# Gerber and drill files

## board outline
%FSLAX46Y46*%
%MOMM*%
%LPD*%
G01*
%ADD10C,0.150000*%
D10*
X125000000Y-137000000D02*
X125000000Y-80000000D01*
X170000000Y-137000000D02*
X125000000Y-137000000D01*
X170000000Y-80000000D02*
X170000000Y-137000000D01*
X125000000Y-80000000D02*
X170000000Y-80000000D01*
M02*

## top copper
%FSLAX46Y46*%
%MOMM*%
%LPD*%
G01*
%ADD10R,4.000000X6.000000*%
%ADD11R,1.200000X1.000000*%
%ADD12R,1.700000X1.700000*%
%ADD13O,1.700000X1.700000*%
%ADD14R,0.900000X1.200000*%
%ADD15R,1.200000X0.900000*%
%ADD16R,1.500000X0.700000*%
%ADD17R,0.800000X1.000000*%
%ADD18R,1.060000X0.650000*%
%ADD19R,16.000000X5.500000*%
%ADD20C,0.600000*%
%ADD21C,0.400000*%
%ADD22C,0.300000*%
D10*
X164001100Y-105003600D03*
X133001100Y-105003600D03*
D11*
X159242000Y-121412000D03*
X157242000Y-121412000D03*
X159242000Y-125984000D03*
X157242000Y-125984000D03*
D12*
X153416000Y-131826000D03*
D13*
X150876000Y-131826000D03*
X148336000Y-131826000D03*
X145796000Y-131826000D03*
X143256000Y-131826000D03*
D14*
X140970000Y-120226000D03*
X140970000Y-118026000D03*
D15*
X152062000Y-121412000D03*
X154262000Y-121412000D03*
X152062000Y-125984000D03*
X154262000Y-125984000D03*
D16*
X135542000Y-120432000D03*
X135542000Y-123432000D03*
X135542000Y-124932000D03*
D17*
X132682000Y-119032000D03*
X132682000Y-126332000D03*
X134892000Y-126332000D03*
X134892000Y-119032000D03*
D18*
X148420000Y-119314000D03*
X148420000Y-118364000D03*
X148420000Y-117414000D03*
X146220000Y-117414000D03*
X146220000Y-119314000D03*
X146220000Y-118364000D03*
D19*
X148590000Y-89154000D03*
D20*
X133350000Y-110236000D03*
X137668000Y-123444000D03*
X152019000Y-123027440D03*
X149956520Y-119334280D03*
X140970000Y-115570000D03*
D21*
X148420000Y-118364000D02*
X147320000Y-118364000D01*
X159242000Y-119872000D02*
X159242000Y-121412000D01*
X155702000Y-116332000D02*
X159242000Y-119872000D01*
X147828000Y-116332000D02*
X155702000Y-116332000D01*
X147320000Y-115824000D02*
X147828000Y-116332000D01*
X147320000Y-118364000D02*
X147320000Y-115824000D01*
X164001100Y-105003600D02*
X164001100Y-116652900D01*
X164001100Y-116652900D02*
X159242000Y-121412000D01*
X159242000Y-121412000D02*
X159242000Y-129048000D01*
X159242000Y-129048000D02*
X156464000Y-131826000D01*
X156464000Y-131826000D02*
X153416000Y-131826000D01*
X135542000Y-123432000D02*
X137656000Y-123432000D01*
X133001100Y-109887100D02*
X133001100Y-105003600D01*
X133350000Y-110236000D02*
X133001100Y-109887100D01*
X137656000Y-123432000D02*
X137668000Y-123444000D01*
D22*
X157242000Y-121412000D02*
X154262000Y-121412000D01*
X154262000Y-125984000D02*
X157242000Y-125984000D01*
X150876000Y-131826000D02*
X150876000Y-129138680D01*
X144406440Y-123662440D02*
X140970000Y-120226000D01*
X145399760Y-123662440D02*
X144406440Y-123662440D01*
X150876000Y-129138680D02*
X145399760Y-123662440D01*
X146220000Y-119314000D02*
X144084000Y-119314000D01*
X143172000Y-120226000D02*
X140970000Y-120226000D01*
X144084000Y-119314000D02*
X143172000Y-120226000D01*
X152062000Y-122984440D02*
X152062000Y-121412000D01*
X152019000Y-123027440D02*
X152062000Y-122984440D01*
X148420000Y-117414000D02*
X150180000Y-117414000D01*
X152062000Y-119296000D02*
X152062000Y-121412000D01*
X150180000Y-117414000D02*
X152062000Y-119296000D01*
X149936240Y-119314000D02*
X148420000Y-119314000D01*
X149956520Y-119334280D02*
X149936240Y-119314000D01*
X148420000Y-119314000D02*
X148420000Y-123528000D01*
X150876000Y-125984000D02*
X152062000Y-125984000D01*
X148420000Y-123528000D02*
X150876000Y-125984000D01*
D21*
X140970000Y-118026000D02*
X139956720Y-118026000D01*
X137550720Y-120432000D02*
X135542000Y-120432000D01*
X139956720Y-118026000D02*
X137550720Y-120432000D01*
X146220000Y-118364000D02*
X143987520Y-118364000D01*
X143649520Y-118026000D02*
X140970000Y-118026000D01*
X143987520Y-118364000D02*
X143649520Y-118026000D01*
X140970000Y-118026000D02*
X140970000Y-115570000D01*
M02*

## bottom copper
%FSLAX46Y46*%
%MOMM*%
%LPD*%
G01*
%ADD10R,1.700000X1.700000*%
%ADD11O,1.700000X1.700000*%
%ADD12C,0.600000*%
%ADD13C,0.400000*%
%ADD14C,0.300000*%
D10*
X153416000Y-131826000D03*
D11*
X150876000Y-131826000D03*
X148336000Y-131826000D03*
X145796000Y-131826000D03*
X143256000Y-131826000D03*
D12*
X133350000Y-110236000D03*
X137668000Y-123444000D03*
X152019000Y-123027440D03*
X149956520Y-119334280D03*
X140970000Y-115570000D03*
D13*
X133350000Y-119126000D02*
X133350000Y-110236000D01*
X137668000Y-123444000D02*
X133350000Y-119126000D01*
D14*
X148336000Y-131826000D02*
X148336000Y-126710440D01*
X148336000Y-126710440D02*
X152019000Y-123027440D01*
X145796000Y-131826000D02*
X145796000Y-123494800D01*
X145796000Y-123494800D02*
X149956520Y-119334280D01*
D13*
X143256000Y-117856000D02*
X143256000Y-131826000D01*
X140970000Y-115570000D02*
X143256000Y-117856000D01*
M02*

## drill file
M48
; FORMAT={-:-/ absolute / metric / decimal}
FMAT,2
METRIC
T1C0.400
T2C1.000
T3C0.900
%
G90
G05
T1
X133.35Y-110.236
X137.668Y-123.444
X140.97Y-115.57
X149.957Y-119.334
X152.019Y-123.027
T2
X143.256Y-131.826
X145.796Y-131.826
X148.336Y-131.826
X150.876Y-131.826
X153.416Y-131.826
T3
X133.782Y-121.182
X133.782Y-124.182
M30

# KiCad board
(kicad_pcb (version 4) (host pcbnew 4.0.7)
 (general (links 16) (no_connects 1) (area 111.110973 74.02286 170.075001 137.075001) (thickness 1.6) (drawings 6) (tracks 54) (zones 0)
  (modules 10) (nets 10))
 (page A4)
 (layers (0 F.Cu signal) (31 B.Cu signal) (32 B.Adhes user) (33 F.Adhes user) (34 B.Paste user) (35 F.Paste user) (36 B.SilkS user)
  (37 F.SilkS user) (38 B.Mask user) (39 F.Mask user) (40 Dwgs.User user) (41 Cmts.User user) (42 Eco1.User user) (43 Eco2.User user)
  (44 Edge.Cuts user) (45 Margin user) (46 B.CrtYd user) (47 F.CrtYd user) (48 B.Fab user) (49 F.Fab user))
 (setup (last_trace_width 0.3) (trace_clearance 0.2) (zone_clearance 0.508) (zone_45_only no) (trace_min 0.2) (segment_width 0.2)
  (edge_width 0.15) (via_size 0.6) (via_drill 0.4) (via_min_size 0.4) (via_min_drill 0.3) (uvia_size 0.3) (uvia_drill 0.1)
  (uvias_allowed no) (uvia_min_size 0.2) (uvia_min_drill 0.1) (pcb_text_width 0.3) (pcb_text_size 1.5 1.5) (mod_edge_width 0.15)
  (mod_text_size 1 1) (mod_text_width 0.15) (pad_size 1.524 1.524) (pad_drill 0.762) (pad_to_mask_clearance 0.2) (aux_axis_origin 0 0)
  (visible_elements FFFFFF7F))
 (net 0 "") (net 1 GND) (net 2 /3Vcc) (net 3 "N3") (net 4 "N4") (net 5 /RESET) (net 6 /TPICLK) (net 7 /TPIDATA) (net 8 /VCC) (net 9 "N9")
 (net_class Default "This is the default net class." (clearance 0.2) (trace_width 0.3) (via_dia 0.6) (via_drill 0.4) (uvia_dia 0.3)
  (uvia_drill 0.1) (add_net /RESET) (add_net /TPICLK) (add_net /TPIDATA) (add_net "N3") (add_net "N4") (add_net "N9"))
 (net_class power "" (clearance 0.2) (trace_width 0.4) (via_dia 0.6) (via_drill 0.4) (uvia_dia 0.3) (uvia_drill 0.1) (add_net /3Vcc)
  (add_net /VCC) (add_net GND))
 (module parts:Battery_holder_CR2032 (layer F.Cu) (at 148.5011 105.0036)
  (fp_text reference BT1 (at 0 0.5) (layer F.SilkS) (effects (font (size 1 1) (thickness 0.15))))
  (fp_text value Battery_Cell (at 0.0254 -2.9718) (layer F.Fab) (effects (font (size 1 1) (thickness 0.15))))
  (pad 2 smd rect (at 15.5 0) (size 4 6) (layers F.Cu F.Paste F.Mask) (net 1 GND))
  (pad 1 smd rect (at -15.5 0) (size 4 6) (layers F.Cu F.Paste F.Mask) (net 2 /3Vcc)))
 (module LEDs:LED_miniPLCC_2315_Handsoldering (layer F.Cu) (at 158.242 121.412 180)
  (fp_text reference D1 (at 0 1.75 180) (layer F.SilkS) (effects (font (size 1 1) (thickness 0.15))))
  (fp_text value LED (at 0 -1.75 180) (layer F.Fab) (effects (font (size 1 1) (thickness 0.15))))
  (pad 1 smd rect (at -1 0) (size 1.2 1) (layers F.Cu F.Paste F.Mask) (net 1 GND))
  (pad 2 smd rect (at 1 0) (size 1.2 1) (layers F.Cu F.Paste F.Mask) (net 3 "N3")))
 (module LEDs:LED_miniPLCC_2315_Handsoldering (layer F.Cu) (at 158.242 125.984 180)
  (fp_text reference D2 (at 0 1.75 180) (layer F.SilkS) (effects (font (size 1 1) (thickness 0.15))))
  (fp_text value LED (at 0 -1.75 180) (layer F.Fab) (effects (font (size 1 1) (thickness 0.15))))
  (pad 1 smd rect (at -1 0) (size 1.2 1) (layers F.Cu F.Paste F.Mask) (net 1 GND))
  (pad 2 smd rect (at 1 0) (size 1.2 1) (layers F.Cu F.Paste F.Mask) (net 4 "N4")))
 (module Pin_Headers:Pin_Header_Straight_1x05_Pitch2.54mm (layer F.Cu) (at 153.416 131.826 270)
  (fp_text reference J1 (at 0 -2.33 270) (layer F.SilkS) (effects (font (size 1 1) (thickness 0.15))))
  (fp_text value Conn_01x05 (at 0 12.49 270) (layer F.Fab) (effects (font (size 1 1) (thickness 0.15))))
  (pad 1 thru_hole rect (at 0 0 270) (size 1.7 1.7) (drill 1) (layers *.Cu *.Mask) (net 1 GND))
  (pad 2 thru_hole oval (at 0 2.54 270) (size 1.7 1.7) (drill 1) (layers *.Cu *.Mask) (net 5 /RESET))
  (pad 3 thru_hole oval (at 0 5.08 270) (size 1.7 1.7) (drill 1) (layers *.Cu *.Mask) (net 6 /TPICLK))
  (pad 4 thru_hole oval (at 0 7.62 270) (size 1.7 1.7) (drill 1) (layers *.Cu *.Mask) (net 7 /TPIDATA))
  (pad 5 thru_hole oval (at 0 10.16 270) (size 1.7 1.7) (drill 1) (layers *.Cu *.Mask) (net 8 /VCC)))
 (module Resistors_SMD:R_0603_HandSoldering (layer F.Cu) (at 140.97 119.126 90)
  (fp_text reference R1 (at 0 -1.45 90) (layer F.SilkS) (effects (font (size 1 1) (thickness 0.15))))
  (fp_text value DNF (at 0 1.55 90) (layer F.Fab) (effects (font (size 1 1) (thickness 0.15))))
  (pad 1 smd rect (at -1.1 0 90) (size 1.2 0.9) (layers F.Cu F.Paste F.Mask) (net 5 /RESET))
  (pad 2 smd rect (at 1.1 0 90) (size 1.2 0.9) (layers F.Cu F.Paste F.Mask) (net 8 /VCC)))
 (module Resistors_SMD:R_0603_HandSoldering (layer F.Cu) (at 153.162 121.412)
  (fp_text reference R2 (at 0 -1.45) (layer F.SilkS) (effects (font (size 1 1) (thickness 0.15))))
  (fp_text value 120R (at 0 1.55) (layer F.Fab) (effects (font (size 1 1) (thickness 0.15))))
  (pad 1 smd rect (at -1.1 0) (size 1.2 0.9) (layers F.Cu F.Paste F.Mask) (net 6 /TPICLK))
  (pad 2 smd rect (at 1.1 0) (size 1.2 0.9) (layers F.Cu F.Paste F.Mask) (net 3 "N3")))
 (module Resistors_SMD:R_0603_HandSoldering (layer F.Cu) (at 153.162 125.984)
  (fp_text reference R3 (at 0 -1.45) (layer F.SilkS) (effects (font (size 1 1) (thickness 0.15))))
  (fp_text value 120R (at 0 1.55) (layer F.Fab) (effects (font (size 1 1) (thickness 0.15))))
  (pad 1 smd rect (at -1.1 0) (size 1.2 0.9) (layers F.Cu F.Paste F.Mask) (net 7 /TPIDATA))
  (pad 2 smd rect (at 1.1 0) (size 1.2 0.9) (layers F.Cu F.Paste F.Mask) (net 4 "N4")))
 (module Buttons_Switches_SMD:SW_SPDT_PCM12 (layer F.Cu) (at 134.112 122.682 270)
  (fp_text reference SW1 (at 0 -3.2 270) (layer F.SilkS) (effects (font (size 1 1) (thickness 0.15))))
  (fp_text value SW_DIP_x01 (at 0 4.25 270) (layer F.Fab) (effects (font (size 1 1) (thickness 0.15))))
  (pad "" np_thru_hole circle (at -1.5 0.33 270) (size 0.9 0.9) (drill 0.9) (layers *.Cu *.Mask))
  (pad "" np_thru_hole circle (at 1.5 0.33 270) (size 0.9 0.9) (drill 0.9) (layers *.Cu *.Mask))
  (pad 1 smd rect (at -2.25 -1.43 270) (size 0.7 1.5) (layers F.Cu F.Paste F.Mask) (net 8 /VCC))
  (pad 2 smd rect (at 0.75 -1.43 270) (size 0.7 1.5) (layers F.Cu F.Paste F.Mask) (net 2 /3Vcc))
  (pad 3 smd rect (at 2.25 -1.43 270) (size 0.7 1.5) (layers F.Cu F.Paste F.Mask))
  (pad "" smd rect (at -3.65 1.43 270) (size 1 0.8) (layers F.Cu F.Paste F.Mask))
  (pad "" smd rect (at 3.65 1.43 270) (size 1 0.8) (layers F.Cu F.Paste F.Mask))
  (pad "" smd rect (at 3.65 -0.78 270) (size 1 0.8) (layers F.Cu F.Paste F.Mask))
  (pad "" smd rect (at -3.65 -0.78 270) (size 1 0.8) (layers F.Cu F.Paste F.Mask)))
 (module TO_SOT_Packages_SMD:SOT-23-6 (layer F.Cu) (at 147.32 118.364 180)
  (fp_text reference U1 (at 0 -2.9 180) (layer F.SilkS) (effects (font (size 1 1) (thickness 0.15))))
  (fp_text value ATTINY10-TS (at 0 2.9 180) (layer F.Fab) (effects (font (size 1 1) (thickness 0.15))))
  (pad 1 smd rect (at -1.1 -0.95 180) (size 1.06 0.65) (layers F.Cu F.Paste F.Mask) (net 7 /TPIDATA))
  (pad 2 smd rect (at -1.1 0 180) (size 1.06 0.65) (layers F.Cu F.Paste F.Mask) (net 1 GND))
  (pad 3 smd rect (at -1.1 0.95 180) (size 1.06 0.65) (layers F.Cu F.Paste F.Mask) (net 6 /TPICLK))
  (pad 4 smd rect (at 1.1 0.95 180) (size 1.06 0.65) (layers F.Cu F.Paste F.Mask) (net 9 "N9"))
  (pad 6 smd rect (at 1.1 -0.95 180) (size 1.06 0.65) (layers F.Cu F.Paste F.Mask) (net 5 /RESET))
  (pad 5 smd rect (at 1.1 0 180) (size 1.06 0.65) (layers F.Cu F.Paste F.Mask) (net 8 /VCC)))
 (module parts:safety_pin (layer F.Cu) (at 148.59 89.154)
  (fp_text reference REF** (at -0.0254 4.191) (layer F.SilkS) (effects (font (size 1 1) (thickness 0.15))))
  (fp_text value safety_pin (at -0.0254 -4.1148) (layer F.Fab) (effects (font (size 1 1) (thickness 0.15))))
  (pad 1 smd rect (at 0 0) (size 16 5.5) (layers F.Cu F.Paste F.Mask)))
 (gr_line (start 125 137) (end 125 80) (angle 90) (layer Edge.Cuts) (width 0.15))
 (gr_line (start 170 137) (end 125 137) (angle 90) (layer Edge.Cuts) (width 0.15))
 (gr_line (start 170 80) (end 170 137) (angle 90) (layer Edge.Cuts) (width 0.15))
 (gr_line (start 125 80) (end 170 80) (angle 90) (layer Edge.Cuts) (width 0.15))
 (segment (start 148.42 118.364) (end 147.32 118.364) (width 0.4) (layer F.Cu) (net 1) (status 400000))
 (segment (start 159.242 119.872) (end 159.242 121.412) (width 0.4) (layer F.Cu) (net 1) (status 800000))
 (segment (start 155.702 116.332) (end 159.242 119.872) (width 0.4) (layer F.Cu) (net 1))
 (segment (start 147.828 116.332) (end 155.702 116.332) (width 0.4) (layer F.Cu) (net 1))
 (segment (start 147.32 115.824) (end 147.828 116.332) (width 0.4) (layer F.Cu) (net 1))
 (segment (start 147.32 118.364) (end 147.32 115.824) (width 0.4) (layer F.Cu) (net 1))
 (segment (start 164.0011 105.0036) (end 164.0011 116.6529) (width 0.4) (layer F.Cu) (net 1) (status 400000))
 (segment (start 164.0011 116.6529) (end 159.242 121.412) (width 0.4) (layer F.Cu) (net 1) (status 800000))
 (segment (start 159.242 121.412) (end 159.242 129.048) (width 0.4) (layer F.Cu) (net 1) (status 400000))
 (segment (start 159.242 129.048) (end 156.464 131.826) (width 0.4) (layer F.Cu) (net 1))
 (segment (start 156.464 131.826) (end 153.416 131.826) (width 0.4) (layer F.Cu) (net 1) (status 800000))
 (segment (start 135.542 123.432) (end 137.656 123.432) (width 0.4) (layer F.Cu) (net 2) (status 400000))
 (segment (start 133.0011 109.8871) (end 133.0011 105.0036) (width 0.4) (layer F.Cu) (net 2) (status 800000))
 (segment (start 133.35 110.236) (end 133.0011 109.8871) (width 0.4) (layer F.Cu) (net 2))
 (via (at 133.35 110.236) (size 0.6) (drill 0.4) (layers F.Cu B.Cu) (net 2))
 (segment (start 133.35 119.126) (end 133.35 110.236) (width 0.4) (layer B.Cu) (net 2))
 (segment (start 137.668 123.444) (end 133.35 119.126) (width 0.4) (layer B.Cu) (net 2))
 (via (at 137.668 123.444) (size 0.6) (drill 0.4) (layers F.Cu B.Cu) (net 2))
 (segment (start 137.656 123.432) (end 137.668 123.444) (width 0.4) (layer F.Cu) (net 2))
 (segment (start 157.242 121.412) (end 154.262 121.412) (width 0.3) (layer F.Cu) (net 3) (status C00000))
 (segment (start 154.262 125.984) (end 157.242 125.984) (width 0.3) (layer F.Cu) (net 4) (status C00000))
 (segment (start 150.876 131.826) (end 150.876 129.13868) (width 0.3) (layer F.Cu) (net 5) (status 400000))
 (segment (start 144.40644 123.66244) (end 140.97 120.226) (width 0.3) (layer F.Cu) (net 5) (status 800000))
 (segment (start 145.39976 123.66244) (end 144.40644 123.66244) (width 0.3) (layer F.Cu) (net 5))
 (segment (start 150.876 129.13868) (end 145.39976 123.66244) (width 0.3) (layer F.Cu) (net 5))
 (segment (start 146.22 119.314) (end 144.084 119.314) (width 0.3) (layer F.Cu) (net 5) (status 400000))
 (segment (start 143.172 120.226) (end 140.97 120.226) (width 0.3) (layer F.Cu) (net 5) (status 800000))
 (segment (start 144.084 119.314) (end 143.172 120.226) (width 0.3) (layer F.Cu) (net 5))
 (segment (start 148.336 131.826) (end 148.336 126.71044) (width 0.3) (layer B.Cu) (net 6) (status 400000))
 (segment (start 152.062 122.98444) (end 152.062 121.412) (width 0.3) (layer F.Cu) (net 6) (status 800000))
 (segment (start 152.019 123.02744) (end 152.062 122.98444) (width 0.3) (layer F.Cu) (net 6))
 (via (at 152.019 123.02744) (size 0.6) (drill 0.4) (layers F.Cu B.Cu) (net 6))
 (segment (start 148.336 126.71044) (end 152.019 123.02744) (width 0.3) (layer B.Cu) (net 6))
 (segment (start 148.42 117.414) (end 150.18 117.414) (width 0.3) (layer F.Cu) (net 6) (status 400000))
 (segment (start 152.062 119.296) (end 152.062 121.412) (width 0.3) (layer F.Cu) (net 6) (status 800000))
 (segment (start 150.18 117.414) (end 152.062 119.296) (width 0.3) (layer F.Cu) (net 6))
 (segment (start 145.796 131.826) (end 145.796 123.4948) (width 0.3) (layer B.Cu) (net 7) (status 400000))
 (segment (start 149.93624 119.314) (end 148.42 119.314) (width 0.3) (layer F.Cu) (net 7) (status 800000))
 (segment (start 149.95652 119.33428) (end 149.93624 119.314) (width 0.3) (layer F.Cu) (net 7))
 (via (at 149.95652 119.33428) (size 0.6) (drill 0.4) (layers F.Cu B.Cu) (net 7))
 (segment (start 145.796 123.4948) (end 149.95652 119.33428) (width 0.3) (layer B.Cu) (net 7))
 (segment (start 148.42 119.314) (end 148.42 123.528) (width 0.3) (layer F.Cu) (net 7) (status 400000))
 (segment (start 150.876 125.984) (end 152.062 125.984) (width 0.3) (layer F.Cu) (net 7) (status 800000))
 (segment (start 148.42 123.528) (end 150.876 125.984) (width 0.3) (layer F.Cu) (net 7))
 (segment (start 140.97 118.026) (end 139.95672 118.026) (width 0.4) (layer F.Cu) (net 8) (status 400000))
 (segment (start 137.55072 120.432) (end 135.542 120.432) (width 0.4) (layer F.Cu) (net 8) (status 800000))
 (segment (start 139.95672 118.026) (end 137.55072 120.432) (width 0.4) (layer F.Cu) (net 8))
 (segment (start 146.22 118.364) (end 143.98752 118.364) (width 0.4) (layer F.Cu) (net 8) (status 400000))
 (segment (start 143.64952 118.026) (end 140.97 118.026) (width 0.4) (layer F.Cu) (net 8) (status 800000))
 (segment (start 143.98752 118.364) (end 143.64952 118.026) (width 0.4) (layer F.Cu) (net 8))
 (segment (start 140.97 118.026) (end 140.97 115.57) (width 0.4) (layer F.Cu) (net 8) (status 400000))
 (segment (start 143.256 117.856) (end 143.256 131.826) (width 0.4) (layer B.Cu) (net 8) (status 800000))
 (segment (start 140.97 115.57) (end 143.256 117.856) (width 0.4) (layer B.Cu) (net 8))
 (via (at 140.97 115.57) (size 0.6) (drill 0.4) (layers F.Cu B.Cu) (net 8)))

